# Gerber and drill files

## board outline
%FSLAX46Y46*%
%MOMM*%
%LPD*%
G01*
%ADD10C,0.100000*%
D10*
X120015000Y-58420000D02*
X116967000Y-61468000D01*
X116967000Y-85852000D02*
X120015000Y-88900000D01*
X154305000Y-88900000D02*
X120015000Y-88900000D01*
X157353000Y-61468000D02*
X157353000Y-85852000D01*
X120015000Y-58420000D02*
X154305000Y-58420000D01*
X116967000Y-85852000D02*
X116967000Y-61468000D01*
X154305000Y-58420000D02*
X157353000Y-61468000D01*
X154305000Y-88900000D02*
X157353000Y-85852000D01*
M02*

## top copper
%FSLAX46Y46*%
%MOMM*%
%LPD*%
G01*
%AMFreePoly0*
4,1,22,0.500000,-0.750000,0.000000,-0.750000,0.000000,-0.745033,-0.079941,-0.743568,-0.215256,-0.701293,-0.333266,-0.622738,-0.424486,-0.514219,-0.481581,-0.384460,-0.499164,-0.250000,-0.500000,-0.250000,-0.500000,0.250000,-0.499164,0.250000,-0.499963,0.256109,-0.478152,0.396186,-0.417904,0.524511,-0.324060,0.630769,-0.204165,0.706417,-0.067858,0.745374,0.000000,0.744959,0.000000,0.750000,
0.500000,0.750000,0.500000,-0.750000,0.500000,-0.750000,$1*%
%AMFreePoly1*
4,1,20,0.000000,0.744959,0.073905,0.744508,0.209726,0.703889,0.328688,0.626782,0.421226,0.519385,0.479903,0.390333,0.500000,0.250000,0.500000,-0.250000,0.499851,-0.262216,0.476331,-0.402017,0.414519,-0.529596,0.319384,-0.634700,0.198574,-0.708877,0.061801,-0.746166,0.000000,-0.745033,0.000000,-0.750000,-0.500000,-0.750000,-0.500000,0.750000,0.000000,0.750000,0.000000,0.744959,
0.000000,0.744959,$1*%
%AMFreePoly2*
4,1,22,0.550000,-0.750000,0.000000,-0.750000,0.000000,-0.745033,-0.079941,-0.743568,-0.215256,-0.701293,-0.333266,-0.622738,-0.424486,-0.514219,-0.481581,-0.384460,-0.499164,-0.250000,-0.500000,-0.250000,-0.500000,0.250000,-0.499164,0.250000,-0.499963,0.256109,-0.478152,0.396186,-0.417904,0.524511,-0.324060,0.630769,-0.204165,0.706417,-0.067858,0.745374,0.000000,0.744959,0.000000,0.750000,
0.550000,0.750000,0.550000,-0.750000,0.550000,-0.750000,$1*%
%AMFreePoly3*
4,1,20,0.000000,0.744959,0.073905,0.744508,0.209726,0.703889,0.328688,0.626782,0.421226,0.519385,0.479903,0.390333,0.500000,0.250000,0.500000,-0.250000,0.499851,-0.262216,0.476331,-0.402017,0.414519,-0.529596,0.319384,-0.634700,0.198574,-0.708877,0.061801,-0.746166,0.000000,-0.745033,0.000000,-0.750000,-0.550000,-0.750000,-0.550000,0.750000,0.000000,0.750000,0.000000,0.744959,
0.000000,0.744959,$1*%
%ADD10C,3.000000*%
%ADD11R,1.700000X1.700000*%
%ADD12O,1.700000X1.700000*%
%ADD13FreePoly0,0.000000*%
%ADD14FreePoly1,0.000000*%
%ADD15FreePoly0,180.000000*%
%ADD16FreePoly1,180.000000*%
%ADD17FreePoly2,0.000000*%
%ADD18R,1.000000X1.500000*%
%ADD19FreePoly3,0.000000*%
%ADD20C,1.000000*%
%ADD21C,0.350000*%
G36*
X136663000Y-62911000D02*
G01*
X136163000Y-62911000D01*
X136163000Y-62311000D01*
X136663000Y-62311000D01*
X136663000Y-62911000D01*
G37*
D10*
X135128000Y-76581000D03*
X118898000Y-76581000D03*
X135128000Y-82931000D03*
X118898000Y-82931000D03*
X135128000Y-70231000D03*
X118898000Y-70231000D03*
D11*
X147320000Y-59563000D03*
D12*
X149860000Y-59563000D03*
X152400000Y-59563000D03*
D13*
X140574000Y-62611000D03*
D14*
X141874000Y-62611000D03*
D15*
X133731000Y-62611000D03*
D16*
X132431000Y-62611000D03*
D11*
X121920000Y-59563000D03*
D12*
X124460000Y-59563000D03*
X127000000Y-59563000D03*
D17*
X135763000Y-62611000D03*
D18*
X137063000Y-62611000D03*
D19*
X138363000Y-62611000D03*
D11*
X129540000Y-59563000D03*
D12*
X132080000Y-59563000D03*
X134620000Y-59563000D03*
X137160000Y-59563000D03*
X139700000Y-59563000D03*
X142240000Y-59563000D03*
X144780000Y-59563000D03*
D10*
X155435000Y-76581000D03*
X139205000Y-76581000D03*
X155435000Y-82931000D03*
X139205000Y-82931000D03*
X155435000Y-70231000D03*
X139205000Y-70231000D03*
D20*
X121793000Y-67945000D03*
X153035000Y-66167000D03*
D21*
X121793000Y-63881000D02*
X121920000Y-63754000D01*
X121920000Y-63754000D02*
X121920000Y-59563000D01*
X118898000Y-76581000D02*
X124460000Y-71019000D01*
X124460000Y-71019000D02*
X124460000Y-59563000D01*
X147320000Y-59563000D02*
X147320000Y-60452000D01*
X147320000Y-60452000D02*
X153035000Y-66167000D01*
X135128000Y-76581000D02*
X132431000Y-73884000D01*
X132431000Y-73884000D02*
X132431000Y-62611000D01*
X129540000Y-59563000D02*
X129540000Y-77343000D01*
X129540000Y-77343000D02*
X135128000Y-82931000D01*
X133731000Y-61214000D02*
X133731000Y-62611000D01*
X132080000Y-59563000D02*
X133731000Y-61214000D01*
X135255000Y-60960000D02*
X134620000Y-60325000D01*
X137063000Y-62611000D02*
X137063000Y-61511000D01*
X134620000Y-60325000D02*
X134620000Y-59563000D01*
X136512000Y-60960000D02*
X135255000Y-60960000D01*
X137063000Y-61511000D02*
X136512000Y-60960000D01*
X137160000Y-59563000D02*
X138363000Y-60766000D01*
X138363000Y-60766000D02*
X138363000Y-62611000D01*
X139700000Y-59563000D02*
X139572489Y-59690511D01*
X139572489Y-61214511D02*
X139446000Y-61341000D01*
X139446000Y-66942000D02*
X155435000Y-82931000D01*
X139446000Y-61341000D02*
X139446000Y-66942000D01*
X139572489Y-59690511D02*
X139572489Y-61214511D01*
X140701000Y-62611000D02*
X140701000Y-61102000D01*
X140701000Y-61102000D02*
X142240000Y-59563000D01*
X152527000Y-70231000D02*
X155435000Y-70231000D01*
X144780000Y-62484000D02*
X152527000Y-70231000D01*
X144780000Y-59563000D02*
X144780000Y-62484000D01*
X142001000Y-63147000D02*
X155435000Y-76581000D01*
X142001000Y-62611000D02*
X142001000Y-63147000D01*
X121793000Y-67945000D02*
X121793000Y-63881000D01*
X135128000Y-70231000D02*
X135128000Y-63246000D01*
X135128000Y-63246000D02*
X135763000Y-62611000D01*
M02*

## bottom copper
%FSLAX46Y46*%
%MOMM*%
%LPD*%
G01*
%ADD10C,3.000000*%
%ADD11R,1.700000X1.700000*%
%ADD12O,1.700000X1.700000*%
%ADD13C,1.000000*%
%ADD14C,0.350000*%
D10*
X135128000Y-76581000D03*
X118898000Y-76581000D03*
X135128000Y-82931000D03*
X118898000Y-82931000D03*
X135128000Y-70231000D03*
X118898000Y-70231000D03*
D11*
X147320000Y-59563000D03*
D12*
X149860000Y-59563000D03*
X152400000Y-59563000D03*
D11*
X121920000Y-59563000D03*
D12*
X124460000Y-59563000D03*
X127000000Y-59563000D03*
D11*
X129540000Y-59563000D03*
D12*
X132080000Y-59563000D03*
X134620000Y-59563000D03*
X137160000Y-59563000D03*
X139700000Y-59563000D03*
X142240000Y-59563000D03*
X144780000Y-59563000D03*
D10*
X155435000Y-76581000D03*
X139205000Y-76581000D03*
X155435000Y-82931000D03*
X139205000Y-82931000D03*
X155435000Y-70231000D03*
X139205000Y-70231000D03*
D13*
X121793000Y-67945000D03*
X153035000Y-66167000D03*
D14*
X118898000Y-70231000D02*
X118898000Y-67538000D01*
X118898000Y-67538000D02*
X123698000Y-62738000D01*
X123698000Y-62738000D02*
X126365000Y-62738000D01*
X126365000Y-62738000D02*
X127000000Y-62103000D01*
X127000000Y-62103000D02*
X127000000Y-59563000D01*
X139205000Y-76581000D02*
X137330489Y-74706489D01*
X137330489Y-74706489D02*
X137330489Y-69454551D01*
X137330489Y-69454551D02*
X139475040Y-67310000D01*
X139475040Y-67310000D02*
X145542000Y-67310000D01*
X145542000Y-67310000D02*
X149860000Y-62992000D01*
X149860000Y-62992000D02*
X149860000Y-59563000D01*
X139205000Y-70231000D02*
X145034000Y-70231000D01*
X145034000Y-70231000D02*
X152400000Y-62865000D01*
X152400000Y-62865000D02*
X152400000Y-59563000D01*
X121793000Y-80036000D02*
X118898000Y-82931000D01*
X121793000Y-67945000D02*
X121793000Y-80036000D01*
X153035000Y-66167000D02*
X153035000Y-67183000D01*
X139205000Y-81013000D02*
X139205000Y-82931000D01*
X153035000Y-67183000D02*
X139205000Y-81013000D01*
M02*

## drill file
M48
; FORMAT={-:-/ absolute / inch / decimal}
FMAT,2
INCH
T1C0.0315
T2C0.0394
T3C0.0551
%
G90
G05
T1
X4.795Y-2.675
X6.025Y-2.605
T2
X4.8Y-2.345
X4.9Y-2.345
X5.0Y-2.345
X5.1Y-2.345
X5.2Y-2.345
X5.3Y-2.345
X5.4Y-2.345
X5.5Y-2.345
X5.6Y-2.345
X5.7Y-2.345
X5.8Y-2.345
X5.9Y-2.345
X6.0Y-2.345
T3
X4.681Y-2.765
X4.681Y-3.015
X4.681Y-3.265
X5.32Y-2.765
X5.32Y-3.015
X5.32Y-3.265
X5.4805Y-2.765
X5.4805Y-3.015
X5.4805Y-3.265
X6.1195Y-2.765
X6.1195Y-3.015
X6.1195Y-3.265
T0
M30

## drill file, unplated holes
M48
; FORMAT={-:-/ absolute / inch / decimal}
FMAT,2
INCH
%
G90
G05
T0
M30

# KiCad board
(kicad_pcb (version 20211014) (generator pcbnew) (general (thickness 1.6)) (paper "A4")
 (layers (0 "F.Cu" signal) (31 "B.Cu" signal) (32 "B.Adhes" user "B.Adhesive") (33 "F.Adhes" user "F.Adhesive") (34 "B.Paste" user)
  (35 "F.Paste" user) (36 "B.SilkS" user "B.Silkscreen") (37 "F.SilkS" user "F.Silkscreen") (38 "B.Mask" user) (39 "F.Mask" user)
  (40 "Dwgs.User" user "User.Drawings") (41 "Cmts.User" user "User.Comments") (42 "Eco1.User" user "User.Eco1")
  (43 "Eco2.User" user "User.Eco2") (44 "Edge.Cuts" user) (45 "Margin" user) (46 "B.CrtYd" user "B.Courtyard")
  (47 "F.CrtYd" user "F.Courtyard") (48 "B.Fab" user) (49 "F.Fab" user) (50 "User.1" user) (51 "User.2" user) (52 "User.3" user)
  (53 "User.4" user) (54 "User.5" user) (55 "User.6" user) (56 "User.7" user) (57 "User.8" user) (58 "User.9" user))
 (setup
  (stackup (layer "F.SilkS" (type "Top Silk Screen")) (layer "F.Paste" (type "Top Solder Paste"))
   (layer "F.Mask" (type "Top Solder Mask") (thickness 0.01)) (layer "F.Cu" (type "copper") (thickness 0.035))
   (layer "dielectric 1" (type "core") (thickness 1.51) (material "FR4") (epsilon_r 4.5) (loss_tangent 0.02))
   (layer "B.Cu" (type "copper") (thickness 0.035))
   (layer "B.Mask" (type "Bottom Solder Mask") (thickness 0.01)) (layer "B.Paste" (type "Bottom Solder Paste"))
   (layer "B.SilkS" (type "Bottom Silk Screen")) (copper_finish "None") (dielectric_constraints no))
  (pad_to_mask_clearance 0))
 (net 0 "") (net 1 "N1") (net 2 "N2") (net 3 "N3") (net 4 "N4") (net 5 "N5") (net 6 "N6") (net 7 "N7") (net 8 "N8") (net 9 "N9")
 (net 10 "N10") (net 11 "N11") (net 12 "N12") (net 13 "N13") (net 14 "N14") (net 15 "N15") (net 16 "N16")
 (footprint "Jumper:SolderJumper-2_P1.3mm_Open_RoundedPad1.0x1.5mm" (layer "F.Cu") (at 141.224 62.611)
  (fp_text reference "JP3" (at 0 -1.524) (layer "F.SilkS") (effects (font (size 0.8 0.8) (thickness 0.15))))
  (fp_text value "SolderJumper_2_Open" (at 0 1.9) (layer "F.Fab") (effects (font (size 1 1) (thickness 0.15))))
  (pad "1" smd custom locked (at -0.65 0) (size 1 0.5) (layers "F.Cu" "F.Mask") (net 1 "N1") (zone_connect 2)
   (options (clearance outline) (anchor rect)) (primitives))
  (pad "2" smd custom locked (at 0.65 0) (size 1 0.5) (layers "F.Cu" "F.Mask") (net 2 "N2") (zone_connect 2)
   (options (clearance outline) (anchor rect)) (primitives)))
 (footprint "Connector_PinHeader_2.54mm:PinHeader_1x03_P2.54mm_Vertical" (layer "F.Cu") (at 147.32 59.563 90)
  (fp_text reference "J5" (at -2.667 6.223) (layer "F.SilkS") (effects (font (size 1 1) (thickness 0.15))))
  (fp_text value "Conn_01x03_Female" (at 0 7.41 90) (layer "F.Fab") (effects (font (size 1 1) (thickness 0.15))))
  (pad "1" thru_hole rect locked (at 0 0 90) (size 1.7 1.7) (drill 1) (layers *.Cu *.Mask) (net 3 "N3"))
  (pad "2" thru_hole oval locked (at 0 2.54 90) (size 1.7 1.7) (drill 1) (layers *.Cu *.Mask) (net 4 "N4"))
  (pad "3" thru_hole oval locked (at 0 5.08 90) (size 1.7 1.7) (drill 1) (layers *.Cu *.Mask) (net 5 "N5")))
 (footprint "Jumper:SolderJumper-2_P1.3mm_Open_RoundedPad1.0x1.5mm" (layer "F.Cu") (at 133.081 62.611 180)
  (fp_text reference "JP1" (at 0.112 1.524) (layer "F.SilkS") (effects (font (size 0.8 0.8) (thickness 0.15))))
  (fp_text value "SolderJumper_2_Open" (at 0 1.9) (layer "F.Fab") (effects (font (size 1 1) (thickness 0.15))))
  (pad "1" smd custom locked (at -0.65 0 180) (size 1 0.5) (layers "F.Cu" "F.Mask") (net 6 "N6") (zone_connect 2)
   (options (clearance outline) (anchor rect)) (primitives))
  (pad "2" smd custom locked (at 0.65 0 180) (size 1 0.5) (layers "F.Cu" "F.Mask") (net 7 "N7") (zone_connect 2)
   (options (clearance outline) (anchor rect)) (primitives)))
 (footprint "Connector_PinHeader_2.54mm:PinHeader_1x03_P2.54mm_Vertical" (layer "F.Cu") (at 121.92 59.563 90)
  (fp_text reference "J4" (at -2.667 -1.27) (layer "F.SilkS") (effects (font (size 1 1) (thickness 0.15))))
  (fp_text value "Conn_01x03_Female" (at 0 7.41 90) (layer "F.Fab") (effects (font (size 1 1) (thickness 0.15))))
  (pad "1" thru_hole rect locked (at 0 0 90) (size 1.7 1.7) (drill 1) (layers *.Cu *.Mask) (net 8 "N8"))
  (pad "2" thru_hole oval locked (at 0 2.54 90) (size 1.7 1.7) (drill 1) (layers *.Cu *.Mask) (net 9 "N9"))
  (pad "3" thru_hole oval locked (at 0 5.08 90) (size 1.7 1.7) (drill 1) (layers *.Cu *.Mask) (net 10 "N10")))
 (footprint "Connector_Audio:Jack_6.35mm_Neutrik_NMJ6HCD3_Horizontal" (layer "F.Cu") (at 135.128 70.231 -90)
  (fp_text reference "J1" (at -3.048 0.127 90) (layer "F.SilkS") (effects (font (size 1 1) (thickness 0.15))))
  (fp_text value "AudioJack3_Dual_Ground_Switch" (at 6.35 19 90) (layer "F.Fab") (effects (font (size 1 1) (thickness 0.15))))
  (pad "R" thru_hole circle locked (at 6.35 0 270) (size 3 3) (drill 1.4) (layers *.Cu *.Mask) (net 7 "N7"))
  (pad "RN" thru_hole circle locked (at 6.35 16.23 270) (size 3 3) (drill 1.4) (layers *.Cu *.Mask) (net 9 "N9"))
  (pad "S" thru_hole circle locked (at 12.7 0 270) (size 3 3) (drill 1.4) (layers *.Cu *.Mask) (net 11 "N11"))
  (pad "SN" thru_hole circle locked (at 12.7 16.23 270) (size 3 3) (drill 1.4) (layers *.Cu *.Mask) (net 8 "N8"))
  (pad "T" thru_hole circle locked (at 0 0 270) (size 3 3) (drill 1.4) (layers *.Cu *.Mask) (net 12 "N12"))
  (pad "TN" thru_hole circle locked (at 0 16.23 270) (size 3 3) (drill 1.4) (layers *.Cu *.Mask) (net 10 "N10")))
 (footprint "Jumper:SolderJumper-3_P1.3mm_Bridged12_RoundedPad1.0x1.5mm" (layer "F.Cu") (at 137.063 62.611)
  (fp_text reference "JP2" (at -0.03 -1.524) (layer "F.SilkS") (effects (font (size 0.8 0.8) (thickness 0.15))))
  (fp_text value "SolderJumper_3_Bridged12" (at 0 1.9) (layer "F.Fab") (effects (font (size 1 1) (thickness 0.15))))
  (fp_poly (pts (xy -0.9 -0.3) (xy -0.4 -0.3) (xy -0.4 0.3) (xy -0.9 0.3)) (layer "F.Cu") (width 0) (fill solid))
  (pad "1" smd custom locked (at -1.3 0) (size 1 0.5) (layers "F.Cu" "F.Mask") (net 12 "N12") (zone_connect 2)
   (options (clearance outline) (anchor rect)) (primitives))
  (pad "2" smd rect locked (at 0 0) (size 1 1.5) (layers "F.Cu" "F.Mask") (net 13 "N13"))
  (pad "3" smd custom locked (at 1.3 0) (size 1 0.5) (layers "F.Cu" "F.Mask") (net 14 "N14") (zone_connect 2)
   (options (clearance outline) (anchor rect)) (primitives)))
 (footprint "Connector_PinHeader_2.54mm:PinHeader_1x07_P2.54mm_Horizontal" (layer "F.Cu") (at 129.54 59.563 90)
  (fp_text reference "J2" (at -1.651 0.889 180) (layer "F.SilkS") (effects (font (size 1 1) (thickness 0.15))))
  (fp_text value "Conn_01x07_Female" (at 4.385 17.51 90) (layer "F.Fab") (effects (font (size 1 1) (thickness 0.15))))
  (pad "1" thru_hole rect locked (at 0 0 90) (size 1.7 1.7) (drill 1) (layers *.Cu *.Mask) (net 11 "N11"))
  (pad "2" thru_hole oval locked (at 0 2.54 90) (size 1.7 1.7) (drill 1) (layers *.Cu *.Mask) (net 6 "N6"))
  (pad "3" thru_hole oval locked (at 0 5.08 90) (size 1.7 1.7) (drill 1) (layers *.Cu *.Mask) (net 13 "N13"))
  (pad "4" thru_hole oval locked (at 0 7.62 90) (size 1.7 1.7) (drill 1) (layers *.Cu *.Mask) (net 14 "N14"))
  (pad "5" thru_hole oval locked (at 0 10.16 90) (size 1.7 1.7) (drill 1) (layers *.Cu *.Mask) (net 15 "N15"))
  (pad "6" thru_hole oval locked (at 0 12.7 90) (size 1.7 1.7) (drill 1) (layers *.Cu *.Mask) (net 1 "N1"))
  (pad "7" thru_hole oval locked (at 0 15.24 90) (size 1.7 1.7) (drill 1) (layers *.Cu *.Mask) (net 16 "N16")))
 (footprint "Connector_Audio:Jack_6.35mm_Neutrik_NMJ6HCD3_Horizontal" (layer "F.Cu") (at 155.435 70.231 -90)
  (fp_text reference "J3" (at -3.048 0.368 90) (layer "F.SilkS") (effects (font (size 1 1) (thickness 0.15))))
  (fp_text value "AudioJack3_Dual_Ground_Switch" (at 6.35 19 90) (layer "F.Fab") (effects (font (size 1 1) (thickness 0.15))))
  (pad "R" thru_hole circle locked (at 6.35 0 270) (size 3 3) (drill 1.4) (layers *.Cu *.Mask) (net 2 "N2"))
  (pad "RN" thru_hole circle locked (at 6.35 16.23 270) (size 3 3) (drill 1.4) (layers *.Cu *.Mask) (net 4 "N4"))
  (pad "S" thru_hole circle locked (at 12.7 0 270) (size 3 3) (drill 1.4) (layers *.Cu *.Mask) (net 15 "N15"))
  (pad "SN" thru_hole circle locked (at 12.7 16.23 270) (size 3 3) (drill 1.4) (layers *.Cu *.Mask) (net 3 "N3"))
  (pad "T" thru_hole circle locked (at 0 0 270) (size 3 3) (drill 1.4) (layers *.Cu *.Mask) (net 16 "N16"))
  (pad "TN" thru_hole circle locked (at 0 16.23 270) (size 3 3) (drill 1.4) (layers *.Cu *.Mask) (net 5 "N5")))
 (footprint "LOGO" (layer "B.Cu") (at 127 81.915 180)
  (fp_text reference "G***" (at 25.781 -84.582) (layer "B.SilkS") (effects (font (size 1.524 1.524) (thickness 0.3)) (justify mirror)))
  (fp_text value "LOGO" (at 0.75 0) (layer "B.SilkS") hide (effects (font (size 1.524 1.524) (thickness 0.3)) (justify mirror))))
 (gr_line (start 120.015 58.42) (end 116.967 61.468) (layer "Edge.Cuts") (width 0.1))
 (gr_line (start 116.967 85.852) (end 120.015 88.9) (layer "Edge.Cuts") (width 0.1))
 (gr_line (start 154.305 88.9) (end 120.015 88.9) (layer "Edge.Cuts") (width 0.1))
 (gr_line (start 157.353 61.468) (end 157.353 85.852) (layer "Edge.Cuts") (width 0.1))
 (gr_line (start 120.015 58.42) (end 154.305 58.42) (layer "Edge.Cuts") (width 0.1))
 (gr_line (start 116.967 85.852) (end 116.967 61.468) (layer "Edge.Cuts") (width 0.1))
 (gr_line (start 154.305 58.42) (end 157.353 61.468) (layer "Edge.Cuts") (width 0.1))
 (gr_line (start 154.305 88.9) (end 157.353 85.852) (layer "Edge.Cuts") (width 0.1))
 (segment (start 135.128 76.581) (end 132.431 73.884) (width 0.35) (layer "F.Cu") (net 7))
 (segment (start 132.431 73.884) (end 132.431 62.611) (width 0.35) (layer "F.Cu") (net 7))
 (segment (start 129.54 59.563) (end 129.54 77.343) (width 0.35) (layer "F.Cu") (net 11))
 (segment (start 129.54 77.343) (end 135.128 82.931) (width 0.35) (layer "F.Cu") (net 11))
 (segment (start 118.898 76.581) (end 124.46 71.019) (width 0.35) (layer "F.Cu") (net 9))
 (segment (start 124.46 71.019) (end 124.46 59.563) (width 0.35) (layer "F.Cu") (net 9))
 (segment (start 133.731 61.214) (end 133.731 62.611) (width 0.35) (layer "F.Cu") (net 6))
 (segment (start 132.08 59.563) (end 133.731 61.214) (width 0.35) (layer "F.Cu") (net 6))
 (segment (start 135.255 60.96) (end 134.62 60.325) (width 0.35) (layer "F.Cu") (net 13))
 (segment (start 137.063 62.611) (end 137.063 61.511) (width 0.35) (layer "F.Cu") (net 13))
 (segment (start 134.62 60.325) (end 134.62 59.563) (width 0.35) (layer "F.Cu") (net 13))
 (segment (start 136.512 60.96) (end 135.255 60.96) (width 0.35) (layer "F.Cu") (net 13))
 (segment (start 137.063 61.511) (end 136.512 60.96) (width 0.35) (layer "F.Cu") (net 13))
 (segment (start 137.16 59.563) (end 138.363 60.766) (width 0.35) (layer "F.Cu") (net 14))
 (segment (start 138.363 60.766) (end 138.363 62.611) (width 0.35) (layer "F.Cu") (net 14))
 (segment (start 139.7 59.563) (end 139.572489 59.690511) (width 0.35) (layer "F.Cu") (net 15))
 (segment (start 139.572489 61.214511) (end 139.446 61.341) (width 0.35) (layer "F.Cu") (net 15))
 (segment (start 139.446 66.942) (end 155.435 82.931) (width 0.35) (layer "F.Cu") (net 15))
 (segment (start 139.446 61.341) (end 139.446 66.942) (width 0.35) (layer "F.Cu") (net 15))
 (segment (start 139.572489 59.690511) (end 139.572489 61.214511) (width 0.35) (layer "F.Cu") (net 15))
 (segment (start 140.701 62.611) (end 140.701 61.102) (width 0.35) (layer "F.Cu") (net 1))
 (segment (start 140.701 61.102) (end 142.24 59.563) (width 0.35) (layer "F.Cu") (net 1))
 (segment (start 152.527 70.231) (end 155.435 70.231) (width 0.35) (layer "F.Cu") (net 16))
 (segment (start 144.78 62.484) (end 152.527 70.231) (width 0.35) (layer "F.Cu") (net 16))
 (segment (start 144.78 59.563) (end 144.78 62.484) (width 0.35) (layer "F.Cu") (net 16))
 (segment (start 142.001 63.147) (end 155.435 76.581) (width 0.35) (layer "F.Cu") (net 2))
 (segment (start 142.001 62.611) (end 142.001 63.147) (width 0.35) (layer "F.Cu") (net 2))
 (segment (start 121.793 67.945) (end 121.793 63.881) (width 0.35) (layer "F.Cu") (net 8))
 (segment (start 121.793 63.881) (end 121.92 63.754) (width 0.35) (layer "F.Cu") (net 8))
 (segment (start 121.92 63.754) (end 121.92 59.563) (width 0.35) (layer "F.Cu") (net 8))
 (via (at 121.793 67.945) (size 1) (drill 0.8) (layers "F.Cu" "B.Cu") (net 8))
 (segment (start 121.793 80.036) (end 118.898 82.931) (width 0.35) (layer "B.Cu") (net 8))
 (segment (start 121.793 67.945) (end 121.793 80.036) (width 0.35) (layer "B.Cu") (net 8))
 (segment (start 135.128 70.231) (end 135.128 63.246) (width 0.35) (layer "F.Cu") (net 12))
 (segment (start 135.128 63.246) (end 135.763 62.611) (width 0.35) (layer "F.Cu") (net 12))
 (segment (start 118.898 70.231) (end 118.898 67.538) (width 0.35) (layer "B.Cu") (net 10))
 (segment (start 126.365 62.738) (end 127 62.103) (width 0.35) (layer "B.Cu") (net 10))
 (segment (start 118.898 67.538) (end 123.698 62.738) (width 0.35) (layer "B.Cu") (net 10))
 (segment (start 123.698 62.738) (end 126.365 62.738) (width 0.35) (layer "B.Cu") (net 10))
 (segment (start 127 62.103) (end 127 59.563) (width 0.35) (layer "B.Cu") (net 10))
 (segment (start 145.542 67.31) (end 149.86 62.992) (width 0.35) (layer "B.Cu") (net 4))
 (segment (start 139.47504 67.31) (end 145.542 67.31) (width 0.35) (layer "B.Cu") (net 4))
 (segment (start 137.330489 69.454551) (end 139.47504 67.31) (width 0.35) (layer "B.Cu") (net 4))
 (segment (start 149.86 62.992) (end 149.86 59.563) (width 0.35) (layer "B.Cu") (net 4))
 (segment (start 139.205 76.581) (end 137.330489 74.706489) (width 0.35) (layer "B.Cu") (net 4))
 (segment (start 137.330489 74.706489) (end 137.330489 69.454551) (width 0.35) (layer "B.Cu") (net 4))
 (segment (start 147.32 59.563) (end 147.32 60.452) (width 0.35) (layer "F.Cu") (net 3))
 (segment (start 147.32 60.452) (end 153.035 66.167) (width 0.35) (layer "F.Cu") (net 3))
 (via (at 153.035 66.167) (size 1) (drill 0.8) (layers "F.Cu" "B.Cu") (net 3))
 (segment (start 153.035 66.167) (end 153.035 67.183) (width 0.35) (layer "B.Cu") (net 3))
 (segment (start 139.205 81.013) (end 139.205 82.931) (width 0.35) (layer "B.Cu") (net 3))
 (segment (start 153.035 67.183) (end 139.205 81.013) (width 0.35) (layer "B.Cu") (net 3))
 (segment (start 139.205 70.231) (end 145.034 70.231) (width 0.35) (layer "B.Cu") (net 5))
 (segment (start 152.4 62.865) (end 152.4 59.563) (width 0.35) (layer "B.Cu") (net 5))
 (segment (start 145.034 70.231) (end 152.4 62.865) (width 0.35) (layer "B.Cu") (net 5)))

